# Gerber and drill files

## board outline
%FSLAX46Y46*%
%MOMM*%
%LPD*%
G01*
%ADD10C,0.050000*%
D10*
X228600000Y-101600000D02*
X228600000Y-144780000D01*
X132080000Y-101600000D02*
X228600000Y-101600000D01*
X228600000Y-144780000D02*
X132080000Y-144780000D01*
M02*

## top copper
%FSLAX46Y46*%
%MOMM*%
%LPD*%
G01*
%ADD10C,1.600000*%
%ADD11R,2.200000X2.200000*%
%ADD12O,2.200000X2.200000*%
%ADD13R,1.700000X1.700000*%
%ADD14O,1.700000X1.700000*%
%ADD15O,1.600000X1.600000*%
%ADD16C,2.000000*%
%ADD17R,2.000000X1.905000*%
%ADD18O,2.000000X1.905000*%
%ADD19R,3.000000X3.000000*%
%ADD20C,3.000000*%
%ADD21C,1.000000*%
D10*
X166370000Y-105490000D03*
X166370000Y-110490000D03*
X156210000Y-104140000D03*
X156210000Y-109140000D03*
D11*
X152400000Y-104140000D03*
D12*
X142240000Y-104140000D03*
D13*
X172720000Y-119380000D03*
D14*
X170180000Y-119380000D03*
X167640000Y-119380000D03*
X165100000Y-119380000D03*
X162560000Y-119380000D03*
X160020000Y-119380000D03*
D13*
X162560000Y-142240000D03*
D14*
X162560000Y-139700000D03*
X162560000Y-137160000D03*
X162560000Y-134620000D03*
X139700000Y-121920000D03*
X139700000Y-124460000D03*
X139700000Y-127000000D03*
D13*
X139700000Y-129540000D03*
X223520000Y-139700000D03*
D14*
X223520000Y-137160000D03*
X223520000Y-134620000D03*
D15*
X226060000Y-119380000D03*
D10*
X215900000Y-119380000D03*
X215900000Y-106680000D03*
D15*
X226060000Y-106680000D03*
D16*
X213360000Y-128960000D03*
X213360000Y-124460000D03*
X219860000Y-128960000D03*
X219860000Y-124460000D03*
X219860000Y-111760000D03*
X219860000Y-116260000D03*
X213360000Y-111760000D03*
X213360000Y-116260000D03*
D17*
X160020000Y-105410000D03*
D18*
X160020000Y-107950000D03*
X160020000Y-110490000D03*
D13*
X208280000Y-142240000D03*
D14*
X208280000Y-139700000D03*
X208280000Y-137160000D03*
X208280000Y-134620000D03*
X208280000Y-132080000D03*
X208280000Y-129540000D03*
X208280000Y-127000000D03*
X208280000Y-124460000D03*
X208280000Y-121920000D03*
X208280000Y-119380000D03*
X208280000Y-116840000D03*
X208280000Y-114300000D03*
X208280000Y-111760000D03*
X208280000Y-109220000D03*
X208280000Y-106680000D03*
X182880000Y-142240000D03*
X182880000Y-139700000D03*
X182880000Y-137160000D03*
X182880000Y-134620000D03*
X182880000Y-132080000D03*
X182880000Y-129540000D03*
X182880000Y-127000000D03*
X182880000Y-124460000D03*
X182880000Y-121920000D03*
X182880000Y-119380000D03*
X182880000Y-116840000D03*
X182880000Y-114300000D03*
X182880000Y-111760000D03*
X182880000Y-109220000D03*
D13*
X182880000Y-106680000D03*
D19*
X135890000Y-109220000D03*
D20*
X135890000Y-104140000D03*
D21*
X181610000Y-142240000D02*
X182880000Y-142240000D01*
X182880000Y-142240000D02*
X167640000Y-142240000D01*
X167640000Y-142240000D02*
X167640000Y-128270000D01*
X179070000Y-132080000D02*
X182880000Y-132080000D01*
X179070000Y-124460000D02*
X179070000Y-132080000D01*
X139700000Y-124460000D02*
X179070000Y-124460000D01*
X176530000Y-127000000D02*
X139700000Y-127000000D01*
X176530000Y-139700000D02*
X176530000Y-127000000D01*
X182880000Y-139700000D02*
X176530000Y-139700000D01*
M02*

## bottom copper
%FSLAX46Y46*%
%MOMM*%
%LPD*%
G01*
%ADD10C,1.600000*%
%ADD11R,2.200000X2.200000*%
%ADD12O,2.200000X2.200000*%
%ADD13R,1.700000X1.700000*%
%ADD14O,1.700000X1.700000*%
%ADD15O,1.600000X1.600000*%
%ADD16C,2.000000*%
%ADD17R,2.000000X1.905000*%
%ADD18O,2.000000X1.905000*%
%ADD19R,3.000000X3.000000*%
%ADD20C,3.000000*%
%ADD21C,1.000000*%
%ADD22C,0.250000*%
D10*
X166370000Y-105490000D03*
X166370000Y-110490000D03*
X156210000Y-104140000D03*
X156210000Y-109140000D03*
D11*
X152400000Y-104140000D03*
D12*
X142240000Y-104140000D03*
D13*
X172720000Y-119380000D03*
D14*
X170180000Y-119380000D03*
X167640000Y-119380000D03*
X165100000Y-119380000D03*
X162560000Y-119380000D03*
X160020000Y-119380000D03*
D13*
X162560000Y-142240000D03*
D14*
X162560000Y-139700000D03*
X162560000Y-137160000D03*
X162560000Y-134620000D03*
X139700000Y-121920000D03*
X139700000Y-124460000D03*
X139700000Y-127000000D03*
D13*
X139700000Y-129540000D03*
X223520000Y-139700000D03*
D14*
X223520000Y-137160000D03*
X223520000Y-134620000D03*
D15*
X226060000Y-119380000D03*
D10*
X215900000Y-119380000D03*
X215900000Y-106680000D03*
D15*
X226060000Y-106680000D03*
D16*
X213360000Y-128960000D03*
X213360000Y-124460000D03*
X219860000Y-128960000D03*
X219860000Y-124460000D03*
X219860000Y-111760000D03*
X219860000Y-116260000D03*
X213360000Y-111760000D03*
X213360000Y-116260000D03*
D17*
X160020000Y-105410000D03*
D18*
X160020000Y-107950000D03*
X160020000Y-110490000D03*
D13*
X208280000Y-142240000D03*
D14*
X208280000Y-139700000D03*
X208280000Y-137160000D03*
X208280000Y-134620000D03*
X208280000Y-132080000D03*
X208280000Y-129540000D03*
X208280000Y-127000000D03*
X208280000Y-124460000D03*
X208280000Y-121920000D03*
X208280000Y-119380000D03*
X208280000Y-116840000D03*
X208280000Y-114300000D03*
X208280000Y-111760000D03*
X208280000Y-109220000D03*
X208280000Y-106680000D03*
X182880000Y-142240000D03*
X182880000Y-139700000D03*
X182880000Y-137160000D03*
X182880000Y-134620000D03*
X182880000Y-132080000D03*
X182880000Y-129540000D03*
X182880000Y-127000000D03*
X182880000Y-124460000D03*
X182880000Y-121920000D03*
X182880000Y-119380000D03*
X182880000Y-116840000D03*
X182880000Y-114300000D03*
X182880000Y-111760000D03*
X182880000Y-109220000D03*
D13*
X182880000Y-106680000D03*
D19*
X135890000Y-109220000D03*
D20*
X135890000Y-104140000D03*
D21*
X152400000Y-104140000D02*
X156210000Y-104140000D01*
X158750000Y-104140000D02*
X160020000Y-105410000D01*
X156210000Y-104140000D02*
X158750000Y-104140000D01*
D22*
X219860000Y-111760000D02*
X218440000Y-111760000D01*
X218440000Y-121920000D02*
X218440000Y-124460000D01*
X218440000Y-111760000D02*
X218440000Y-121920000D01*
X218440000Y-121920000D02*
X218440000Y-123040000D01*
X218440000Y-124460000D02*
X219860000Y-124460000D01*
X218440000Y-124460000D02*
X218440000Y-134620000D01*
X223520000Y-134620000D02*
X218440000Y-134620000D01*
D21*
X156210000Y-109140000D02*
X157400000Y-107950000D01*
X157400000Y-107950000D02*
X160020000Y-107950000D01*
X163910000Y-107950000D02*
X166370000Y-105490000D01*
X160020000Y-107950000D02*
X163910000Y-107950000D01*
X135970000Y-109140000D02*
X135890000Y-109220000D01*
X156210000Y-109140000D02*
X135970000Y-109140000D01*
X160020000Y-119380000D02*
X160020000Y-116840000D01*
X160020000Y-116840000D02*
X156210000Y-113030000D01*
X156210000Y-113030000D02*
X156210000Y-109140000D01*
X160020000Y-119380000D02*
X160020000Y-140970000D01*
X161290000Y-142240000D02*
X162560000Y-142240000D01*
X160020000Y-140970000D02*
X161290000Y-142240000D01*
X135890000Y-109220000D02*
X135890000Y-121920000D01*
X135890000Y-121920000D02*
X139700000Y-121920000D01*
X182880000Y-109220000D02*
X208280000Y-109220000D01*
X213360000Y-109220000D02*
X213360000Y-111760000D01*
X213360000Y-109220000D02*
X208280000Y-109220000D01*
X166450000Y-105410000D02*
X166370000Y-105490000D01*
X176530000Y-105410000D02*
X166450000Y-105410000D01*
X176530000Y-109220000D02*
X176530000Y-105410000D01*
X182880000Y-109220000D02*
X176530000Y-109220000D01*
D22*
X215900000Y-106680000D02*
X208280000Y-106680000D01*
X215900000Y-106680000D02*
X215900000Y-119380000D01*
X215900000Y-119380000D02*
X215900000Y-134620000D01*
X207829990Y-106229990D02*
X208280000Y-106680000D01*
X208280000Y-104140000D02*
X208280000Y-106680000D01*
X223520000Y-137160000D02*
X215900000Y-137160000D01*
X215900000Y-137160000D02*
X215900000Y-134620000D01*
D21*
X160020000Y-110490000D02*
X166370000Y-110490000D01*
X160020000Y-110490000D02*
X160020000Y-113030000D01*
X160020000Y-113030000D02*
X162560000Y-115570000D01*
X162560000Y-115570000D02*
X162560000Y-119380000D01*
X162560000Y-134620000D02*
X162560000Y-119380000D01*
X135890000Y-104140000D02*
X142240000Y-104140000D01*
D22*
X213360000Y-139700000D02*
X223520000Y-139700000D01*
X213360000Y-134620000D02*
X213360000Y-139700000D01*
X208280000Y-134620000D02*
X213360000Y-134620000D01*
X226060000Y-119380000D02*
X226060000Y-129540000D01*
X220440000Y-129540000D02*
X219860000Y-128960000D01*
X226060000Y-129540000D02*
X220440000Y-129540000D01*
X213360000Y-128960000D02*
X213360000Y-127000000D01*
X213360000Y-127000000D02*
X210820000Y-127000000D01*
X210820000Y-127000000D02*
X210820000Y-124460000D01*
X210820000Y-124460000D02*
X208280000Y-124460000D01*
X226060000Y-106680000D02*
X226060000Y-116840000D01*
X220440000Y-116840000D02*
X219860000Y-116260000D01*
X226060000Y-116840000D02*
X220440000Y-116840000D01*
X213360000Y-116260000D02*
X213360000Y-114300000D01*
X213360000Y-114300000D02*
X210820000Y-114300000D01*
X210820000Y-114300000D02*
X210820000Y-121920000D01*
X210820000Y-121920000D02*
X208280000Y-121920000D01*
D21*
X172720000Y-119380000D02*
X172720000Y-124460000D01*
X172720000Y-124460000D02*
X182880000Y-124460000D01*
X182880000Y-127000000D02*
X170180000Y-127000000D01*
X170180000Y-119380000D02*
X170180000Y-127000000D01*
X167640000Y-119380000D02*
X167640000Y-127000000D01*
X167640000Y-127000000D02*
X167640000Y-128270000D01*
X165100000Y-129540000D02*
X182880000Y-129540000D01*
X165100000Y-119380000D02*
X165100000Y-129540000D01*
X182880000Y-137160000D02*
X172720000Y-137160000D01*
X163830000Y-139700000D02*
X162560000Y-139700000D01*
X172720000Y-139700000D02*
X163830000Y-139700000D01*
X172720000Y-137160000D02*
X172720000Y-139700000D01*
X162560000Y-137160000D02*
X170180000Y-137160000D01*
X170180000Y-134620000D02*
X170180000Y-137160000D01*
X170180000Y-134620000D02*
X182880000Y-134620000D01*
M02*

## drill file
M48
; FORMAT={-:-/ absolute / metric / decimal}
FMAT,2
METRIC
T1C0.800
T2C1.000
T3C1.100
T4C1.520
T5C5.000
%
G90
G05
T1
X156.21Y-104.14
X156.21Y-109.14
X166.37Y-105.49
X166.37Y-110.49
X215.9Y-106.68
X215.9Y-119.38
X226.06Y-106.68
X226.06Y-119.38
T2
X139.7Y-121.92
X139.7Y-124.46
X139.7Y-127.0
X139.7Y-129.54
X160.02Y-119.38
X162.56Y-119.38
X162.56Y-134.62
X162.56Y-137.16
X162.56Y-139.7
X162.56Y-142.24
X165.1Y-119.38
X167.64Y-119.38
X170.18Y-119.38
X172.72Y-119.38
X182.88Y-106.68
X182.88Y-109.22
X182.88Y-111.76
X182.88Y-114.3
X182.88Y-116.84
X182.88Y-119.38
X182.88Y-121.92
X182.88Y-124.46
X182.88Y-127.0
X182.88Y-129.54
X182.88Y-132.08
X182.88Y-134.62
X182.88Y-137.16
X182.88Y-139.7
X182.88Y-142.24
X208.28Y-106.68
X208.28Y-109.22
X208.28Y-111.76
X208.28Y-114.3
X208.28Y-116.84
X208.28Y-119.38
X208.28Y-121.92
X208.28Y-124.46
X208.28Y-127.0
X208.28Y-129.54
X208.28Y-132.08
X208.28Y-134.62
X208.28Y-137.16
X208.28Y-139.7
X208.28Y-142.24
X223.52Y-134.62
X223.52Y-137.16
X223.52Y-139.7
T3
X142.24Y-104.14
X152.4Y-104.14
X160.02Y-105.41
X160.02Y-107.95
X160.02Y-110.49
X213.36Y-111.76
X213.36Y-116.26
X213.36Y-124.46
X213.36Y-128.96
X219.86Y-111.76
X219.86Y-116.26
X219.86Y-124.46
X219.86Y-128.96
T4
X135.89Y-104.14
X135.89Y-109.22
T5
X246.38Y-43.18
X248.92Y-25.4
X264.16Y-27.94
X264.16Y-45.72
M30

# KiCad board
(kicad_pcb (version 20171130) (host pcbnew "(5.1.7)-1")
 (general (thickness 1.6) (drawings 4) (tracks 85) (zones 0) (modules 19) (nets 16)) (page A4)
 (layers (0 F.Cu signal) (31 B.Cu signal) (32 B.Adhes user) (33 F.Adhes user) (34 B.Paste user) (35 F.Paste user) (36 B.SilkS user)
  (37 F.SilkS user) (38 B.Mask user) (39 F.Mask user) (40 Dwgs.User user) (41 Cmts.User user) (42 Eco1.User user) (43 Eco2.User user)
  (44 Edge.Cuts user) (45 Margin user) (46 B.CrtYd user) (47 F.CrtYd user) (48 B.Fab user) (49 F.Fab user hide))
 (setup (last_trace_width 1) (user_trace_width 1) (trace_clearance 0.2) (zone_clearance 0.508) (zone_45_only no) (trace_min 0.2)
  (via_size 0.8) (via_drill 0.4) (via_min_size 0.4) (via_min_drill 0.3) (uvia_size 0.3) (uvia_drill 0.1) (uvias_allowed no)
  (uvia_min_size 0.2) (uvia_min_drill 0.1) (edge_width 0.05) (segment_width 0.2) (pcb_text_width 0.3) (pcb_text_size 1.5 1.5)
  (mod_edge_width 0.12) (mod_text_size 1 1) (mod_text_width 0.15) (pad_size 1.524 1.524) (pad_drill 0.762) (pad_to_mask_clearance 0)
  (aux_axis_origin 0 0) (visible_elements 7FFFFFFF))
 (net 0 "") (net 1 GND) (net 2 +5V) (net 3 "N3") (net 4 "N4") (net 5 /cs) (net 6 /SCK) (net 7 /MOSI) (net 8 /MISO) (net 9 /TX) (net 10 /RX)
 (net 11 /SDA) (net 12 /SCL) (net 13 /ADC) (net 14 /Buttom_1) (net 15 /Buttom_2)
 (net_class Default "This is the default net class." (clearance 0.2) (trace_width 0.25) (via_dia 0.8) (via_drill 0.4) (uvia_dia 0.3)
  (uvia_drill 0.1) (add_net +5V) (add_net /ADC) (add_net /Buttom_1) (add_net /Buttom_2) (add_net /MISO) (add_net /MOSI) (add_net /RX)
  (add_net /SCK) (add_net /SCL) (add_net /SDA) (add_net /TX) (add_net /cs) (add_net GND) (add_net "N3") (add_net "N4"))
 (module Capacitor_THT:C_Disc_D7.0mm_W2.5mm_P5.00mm (layer F.Cu) (at 166.37 110.49 90)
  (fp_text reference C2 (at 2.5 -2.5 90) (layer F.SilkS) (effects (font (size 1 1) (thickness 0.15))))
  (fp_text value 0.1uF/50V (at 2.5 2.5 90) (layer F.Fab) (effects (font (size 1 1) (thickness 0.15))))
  (pad 2 thru_hole circle (at 5 0 90) (size 1.6 1.6) (drill 0.8) (layers *.Cu *.Mask) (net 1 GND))
  (pad 1 thru_hole circle (at 0 0 90) (size 1.6 1.6) (drill 0.8) (layers *.Cu *.Mask) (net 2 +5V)))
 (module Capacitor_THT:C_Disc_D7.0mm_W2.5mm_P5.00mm (layer F.Cu) (at 156.21 104.14 270)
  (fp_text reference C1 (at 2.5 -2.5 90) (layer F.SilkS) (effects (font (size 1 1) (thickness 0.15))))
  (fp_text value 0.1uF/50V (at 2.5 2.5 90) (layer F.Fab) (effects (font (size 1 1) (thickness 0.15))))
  (pad 1 thru_hole circle (at 0 0 270) (size 1.6 1.6) (drill 0.8) (layers *.Cu *.Mask) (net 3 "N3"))
  (pad 2 thru_hole circle (at 5 0 270) (size 1.6 1.6) (drill 0.8) (layers *.Cu *.Mask) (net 1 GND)))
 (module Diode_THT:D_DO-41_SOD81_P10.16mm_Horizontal (layer F.Cu) (at 152.4 104.14 180)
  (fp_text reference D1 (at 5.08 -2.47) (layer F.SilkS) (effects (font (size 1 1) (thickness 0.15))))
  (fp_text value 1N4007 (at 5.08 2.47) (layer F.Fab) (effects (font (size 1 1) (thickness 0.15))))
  (pad 1 thru_hole rect (at 0 0 180) (size 2.2 2.2) (drill 1.1) (layers *.Cu *.Mask) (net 3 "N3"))
  (pad 2 thru_hole oval (at 10.16 0 180) (size 2.2 2.2) (drill 1.1) (layers *.Cu *.Mask) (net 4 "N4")))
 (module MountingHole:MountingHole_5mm (layer F.Cu) (at 248.92 25.4)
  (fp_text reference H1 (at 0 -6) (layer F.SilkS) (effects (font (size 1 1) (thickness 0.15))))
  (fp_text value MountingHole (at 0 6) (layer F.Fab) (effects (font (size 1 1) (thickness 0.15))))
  (pad 1 np_thru_hole circle (at 0 0) (size 5 5) (drill 5) (layers *.Cu *.Mask)))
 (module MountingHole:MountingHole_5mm (layer F.Cu) (at 264.16 45.72)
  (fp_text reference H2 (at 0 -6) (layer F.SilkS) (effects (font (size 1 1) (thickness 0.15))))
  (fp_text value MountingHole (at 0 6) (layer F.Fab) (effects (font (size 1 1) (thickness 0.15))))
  (pad 1 np_thru_hole circle (at 0 0) (size 5 5) (drill 5) (layers *.Cu *.Mask)))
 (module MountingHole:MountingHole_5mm (layer F.Cu) (at 264.16 27.94)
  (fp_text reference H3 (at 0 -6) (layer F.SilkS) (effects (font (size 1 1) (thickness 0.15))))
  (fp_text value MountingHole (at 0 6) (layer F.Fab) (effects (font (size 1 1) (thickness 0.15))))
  (pad 1 np_thru_hole circle (at 0 0) (size 5 5) (drill 5) (layers *.Cu *.Mask)))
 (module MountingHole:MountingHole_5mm (layer F.Cu) (at 246.38 43.18)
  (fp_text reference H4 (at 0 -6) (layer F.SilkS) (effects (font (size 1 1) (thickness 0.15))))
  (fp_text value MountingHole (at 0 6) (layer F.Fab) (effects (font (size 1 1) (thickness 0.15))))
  (pad 1 np_thru_hole circle (at 0 0) (size 5 5) (drill 5) (layers *.Cu *.Mask)))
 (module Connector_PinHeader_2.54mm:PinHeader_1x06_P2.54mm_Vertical (layer F.Cu) (at 172.72 119.38 270)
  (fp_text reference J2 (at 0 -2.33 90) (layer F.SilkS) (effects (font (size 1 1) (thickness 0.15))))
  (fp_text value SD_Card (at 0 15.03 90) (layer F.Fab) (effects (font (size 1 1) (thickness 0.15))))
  (pad 1 thru_hole rect (at 0 0 270) (size 1.7 1.7) (drill 1) (layers *.Cu *.Mask) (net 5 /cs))
  (pad 2 thru_hole oval (at 0 2.54 270) (size 1.7 1.7) (drill 1) (layers *.Cu *.Mask) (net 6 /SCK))
  (pad 3 thru_hole oval (at 0 5.08 270) (size 1.7 1.7) (drill 1) (layers *.Cu *.Mask) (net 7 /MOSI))
  (pad 4 thru_hole oval (at 0 7.62 270) (size 1.7 1.7) (drill 1) (layers *.Cu *.Mask) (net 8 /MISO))
  (pad 5 thru_hole oval (at 0 10.16 270) (size 1.7 1.7) (drill 1) (layers *.Cu *.Mask) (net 2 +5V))
  (pad 6 thru_hole oval (at 0 12.7 270) (size 1.7 1.7) (drill 1) (layers *.Cu *.Mask) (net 1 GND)))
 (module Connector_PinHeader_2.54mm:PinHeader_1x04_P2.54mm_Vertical (layer F.Cu) (at 162.56 142.24 180)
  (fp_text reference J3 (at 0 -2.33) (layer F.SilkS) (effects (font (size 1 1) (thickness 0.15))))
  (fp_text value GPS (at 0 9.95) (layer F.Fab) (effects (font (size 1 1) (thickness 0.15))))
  (pad 1 thru_hole rect (at 0 0 180) (size 1.7 1.7) (drill 1) (layers *.Cu *.Mask) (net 1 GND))
  (pad 2 thru_hole oval (at 0 2.54 180) (size 1.7 1.7) (drill 1) (layers *.Cu *.Mask) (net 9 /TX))
  (pad 3 thru_hole oval (at 0 5.08 180) (size 1.7 1.7) (drill 1) (layers *.Cu *.Mask) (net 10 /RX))
  (pad 4 thru_hole oval (at 0 7.62 180) (size 1.7 1.7) (drill 1) (layers *.Cu *.Mask) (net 2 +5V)))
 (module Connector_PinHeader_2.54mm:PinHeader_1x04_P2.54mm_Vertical (layer F.Cu) (at 139.7 129.54 180)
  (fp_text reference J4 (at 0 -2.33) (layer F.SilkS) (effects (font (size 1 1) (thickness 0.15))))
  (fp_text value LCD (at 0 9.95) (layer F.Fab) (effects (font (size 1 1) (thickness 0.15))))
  (pad 4 thru_hole oval (at 0 7.62 180) (size 1.7 1.7) (drill 1) (layers *.Cu *.Mask) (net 1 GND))
  (pad 3 thru_hole oval (at 0 5.08 180) (size 1.7 1.7) (drill 1) (layers *.Cu *.Mask) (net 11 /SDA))
  (pad 2 thru_hole oval (at 0 2.54 180) (size 1.7 1.7) (drill 1) (layers *.Cu *.Mask) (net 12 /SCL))
  (pad 1 thru_hole rect (at 0 0 180) (size 1.7 1.7) (drill 1) (layers *.Cu *.Mask) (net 2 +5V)))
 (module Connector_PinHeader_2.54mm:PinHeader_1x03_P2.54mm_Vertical (layer F.Cu) (at 223.52 139.7 180)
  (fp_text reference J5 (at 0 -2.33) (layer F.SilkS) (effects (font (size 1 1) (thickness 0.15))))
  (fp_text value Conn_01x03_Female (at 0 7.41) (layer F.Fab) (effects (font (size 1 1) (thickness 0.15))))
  (pad 1 thru_hole rect (at 0 0 180) (size 1.7 1.7) (drill 1) (layers *.Cu *.Mask) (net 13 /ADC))
  (pad 2 thru_hole oval (at 0 2.54 180) (size 1.7 1.7) (drill 1) (layers *.Cu *.Mask) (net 2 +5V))
  (pad 3 thru_hole oval (at 0 5.08 180) (size 1.7 1.7) (drill 1) (layers *.Cu *.Mask) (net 1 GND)))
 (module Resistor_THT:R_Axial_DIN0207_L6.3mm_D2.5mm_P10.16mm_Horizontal (layer F.Cu) (at 215.9 119.38)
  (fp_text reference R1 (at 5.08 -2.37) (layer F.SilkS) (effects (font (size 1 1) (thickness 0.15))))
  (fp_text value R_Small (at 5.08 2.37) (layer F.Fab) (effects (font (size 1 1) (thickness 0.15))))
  (pad 2 thru_hole oval (at 10.16 0) (size 1.6 1.6) (drill 0.8) (layers *.Cu *.Mask) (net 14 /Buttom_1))
  (pad 1 thru_hole circle (at 0 0) (size 1.6 1.6) (drill 0.8) (layers *.Cu *.Mask) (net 2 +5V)))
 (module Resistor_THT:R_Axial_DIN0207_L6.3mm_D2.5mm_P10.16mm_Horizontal (layer F.Cu) (at 215.9 106.68)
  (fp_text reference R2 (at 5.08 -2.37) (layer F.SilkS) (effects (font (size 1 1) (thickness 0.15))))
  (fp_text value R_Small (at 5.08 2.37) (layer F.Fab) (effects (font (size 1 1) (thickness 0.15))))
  (pad 1 thru_hole circle (at 0 0) (size 1.6 1.6) (drill 0.8) (layers *.Cu *.Mask) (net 2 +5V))
  (pad 2 thru_hole oval (at 10.16 0) (size 1.6 1.6) (drill 0.8) (layers *.Cu *.Mask) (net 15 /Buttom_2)))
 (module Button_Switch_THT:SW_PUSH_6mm (layer F.Cu) (at 213.36 124.46)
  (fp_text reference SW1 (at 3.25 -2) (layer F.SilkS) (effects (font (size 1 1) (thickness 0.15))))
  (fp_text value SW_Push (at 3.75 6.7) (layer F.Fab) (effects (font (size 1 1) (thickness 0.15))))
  (pad 2 thru_hole circle (at 0 4.5 90) (size 2 2) (drill 1.1) (layers *.Cu *.Mask) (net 14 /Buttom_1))
  (pad 1 thru_hole circle (at 0 0 90) (size 2 2) (drill 1.1) (layers *.Cu *.Mask) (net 1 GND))
  (pad 2 thru_hole circle (at 6.5 4.5 90) (size 2 2) (drill 1.1) (layers *.Cu *.Mask) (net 14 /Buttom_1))
  (pad 1 thru_hole circle (at 6.5 0 90) (size 2 2) (drill 1.1) (layers *.Cu *.Mask) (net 1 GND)))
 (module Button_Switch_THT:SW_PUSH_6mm (layer F.Cu) (at 213.36 111.76)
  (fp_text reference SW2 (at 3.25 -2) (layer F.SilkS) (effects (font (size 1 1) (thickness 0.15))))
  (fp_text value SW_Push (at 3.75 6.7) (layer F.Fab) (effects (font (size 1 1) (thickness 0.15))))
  (pad 1 thru_hole circle (at 6.5 0 90) (size 2 2) (drill 1.1) (layers *.Cu *.Mask) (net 1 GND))
  (pad 2 thru_hole circle (at 6.5 4.5 90) (size 2 2) (drill 1.1) (layers *.Cu *.Mask) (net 15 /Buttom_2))
  (pad 1 thru_hole circle (at 0 0 90) (size 2 2) (drill 1.1) (layers *.Cu *.Mask) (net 1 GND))
  (pad 2 thru_hole circle (at 0 4.5 90) (size 2 2) (drill 1.1) (layers *.Cu *.Mask) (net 15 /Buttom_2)))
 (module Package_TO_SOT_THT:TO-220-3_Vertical (layer F.Cu) (at 160.02 105.41 270)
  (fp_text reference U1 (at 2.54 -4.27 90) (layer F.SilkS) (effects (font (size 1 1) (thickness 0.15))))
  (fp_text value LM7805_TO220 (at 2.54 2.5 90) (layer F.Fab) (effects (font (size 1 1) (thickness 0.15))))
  (pad 1 thru_hole rect (at 0 0 270) (size 1.905 2) (drill 1.1) (layers *.Cu *.Mask) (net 3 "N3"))
  (pad 2 thru_hole oval (at 2.54 0 270) (size 1.905 2) (drill 1.1) (layers *.Cu *.Mask) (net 1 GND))
  (pad 3 thru_hole oval (at 5.08 0 270) (size 1.905 2) (drill 1.1) (layers *.Cu *.Mask) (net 2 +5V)))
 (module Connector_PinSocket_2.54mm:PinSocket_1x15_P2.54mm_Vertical (layer F.Cu) (at 208.28 142.24 180)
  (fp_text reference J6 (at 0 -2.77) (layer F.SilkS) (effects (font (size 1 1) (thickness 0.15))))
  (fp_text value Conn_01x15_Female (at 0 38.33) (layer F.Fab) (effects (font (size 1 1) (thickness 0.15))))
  (pad 1 thru_hole rect (at 0 0 180) (size 1.7 1.7) (drill 1) (layers *.Cu *.Mask))
  (pad 2 thru_hole oval (at 0 2.54 180) (size 1.7 1.7) (drill 1) (layers *.Cu *.Mask))
  (pad 3 thru_hole oval (at 0 5.08 180) (size 1.7 1.7) (drill 1) (layers *.Cu *.Mask))
  (pad 4 thru_hole oval (at 0 7.62 180) (size 1.7 1.7) (drill 1) (layers *.Cu *.Mask) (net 13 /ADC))
  (pad 5 thru_hole oval (at 0 10.16 180) (size 1.7 1.7) (drill 1) (layers *.Cu *.Mask))
  (pad 6 thru_hole oval (at 0 12.7 180) (size 1.7 1.7) (drill 1) (layers *.Cu *.Mask))
  (pad 7 thru_hole oval (at 0 15.24 180) (size 1.7 1.7) (drill 1) (layers *.Cu *.Mask))
  (pad 8 thru_hole oval (at 0 17.78 180) (size 1.7 1.7) (drill 1) (layers *.Cu *.Mask) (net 14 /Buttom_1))
  (pad 9 thru_hole oval (at 0 20.32 180) (size 1.7 1.7) (drill 1) (layers *.Cu *.Mask) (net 15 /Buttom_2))
  (pad 10 thru_hole oval (at 0 22.86 180) (size 1.7 1.7) (drill 1) (layers *.Cu *.Mask))
  (pad 11 thru_hole oval (at 0 25.4 180) (size 1.7 1.7) (drill 1) (layers *.Cu *.Mask))
  (pad 12 thru_hole oval (at 0 27.94 180) (size 1.7 1.7) (drill 1) (layers *.Cu *.Mask))
  (pad 13 thru_hole oval (at 0 30.48 180) (size 1.7 1.7) (drill 1) (layers *.Cu *.Mask))
  (pad 14 thru_hole oval (at 0 33.02 180) (size 1.7 1.7) (drill 1) (layers *.Cu *.Mask) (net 1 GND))
  (pad 15 thru_hole oval (at 0 35.56 180) (size 1.7 1.7) (drill 1) (layers *.Cu *.Mask) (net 2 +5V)))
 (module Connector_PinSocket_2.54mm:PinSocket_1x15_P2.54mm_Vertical (layer F.Cu) (at 182.88 106.68)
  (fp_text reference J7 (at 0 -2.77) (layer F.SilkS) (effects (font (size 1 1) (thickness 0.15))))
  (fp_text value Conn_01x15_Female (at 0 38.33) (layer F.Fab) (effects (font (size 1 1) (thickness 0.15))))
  (pad 15 thru_hole oval (at 0 35.56) (size 1.7 1.7) (drill 1) (layers *.Cu *.Mask) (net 7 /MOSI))
  (pad 14 thru_hole oval (at 0 33.02) (size 1.7 1.7) (drill 1) (layers *.Cu *.Mask) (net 12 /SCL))
  (pad 13 thru_hole oval (at 0 30.48) (size 1.7 1.7) (drill 1) (layers *.Cu *.Mask) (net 9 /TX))
  (pad 12 thru_hole oval (at 0 27.94) (size 1.7 1.7) (drill 1) (layers *.Cu *.Mask) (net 10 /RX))
  (pad 11 thru_hole oval (at 0 25.4) (size 1.7 1.7) (drill 1) (layers *.Cu *.Mask) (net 11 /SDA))
  (pad 10 thru_hole oval (at 0 22.86) (size 1.7 1.7) (drill 1) (layers *.Cu *.Mask) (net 8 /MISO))
  (pad 9 thru_hole oval (at 0 20.32) (size 1.7 1.7) (drill 1) (layers *.Cu *.Mask) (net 6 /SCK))
  (pad 8 thru_hole oval (at 0 17.78) (size 1.7 1.7) (drill 1) (layers *.Cu *.Mask) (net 5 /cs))
  (pad 7 thru_hole oval (at 0 15.24) (size 1.7 1.7) (drill 1) (layers *.Cu *.Mask))
  (pad 6 thru_hole oval (at 0 12.7) (size 1.7 1.7) (drill 1) (layers *.Cu *.Mask))
  (pad 5 thru_hole oval (at 0 10.16) (size 1.7 1.7) (drill 1) (layers *.Cu *.Mask))
  (pad 4 thru_hole oval (at 0 7.62) (size 1.7 1.7) (drill 1) (layers *.Cu *.Mask))
  (pad 3 thru_hole oval (at 0 5.08) (size 1.7 1.7) (drill 1) (layers *.Cu *.Mask))
  (pad 2 thru_hole oval (at 0 2.54) (size 1.7 1.7) (drill 1) (layers *.Cu *.Mask) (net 1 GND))
  (pad 1 thru_hole rect (at 0 0) (size 1.7 1.7) (drill 1) (layers *.Cu *.Mask)))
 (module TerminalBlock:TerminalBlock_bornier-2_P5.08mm (layer F.Cu) (at 135.89 109.22 90)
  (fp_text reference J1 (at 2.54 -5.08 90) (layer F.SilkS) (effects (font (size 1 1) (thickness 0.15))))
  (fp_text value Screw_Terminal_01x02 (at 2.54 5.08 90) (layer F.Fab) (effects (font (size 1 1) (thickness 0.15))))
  (pad 1 thru_hole rect (at 0 0 90) (size 3 3) (drill 1.52) (layers *.Cu *.Mask) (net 1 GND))
  (pad 2 thru_hole circle (at 5.08 0 90) (size 3 3) (drill 1.52) (layers *.Cu *.Mask) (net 4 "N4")))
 (gr_line (start 228.6 101.6) (end 228.6 144.78) (layer Edge.Cuts) (width 0.05))
 (gr_line (start 132.08 101.6) (end 228.6 101.6) (layer Edge.Cuts) (width 0.05))
 (gr_line (start 228.6 144.78) (end 132.08 144.78) (layer Edge.Cuts) (width 0.05))
 (segment (start 152.4 104.14) (end 156.21 104.14) (width 1) (layer B.Cu) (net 3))
 (segment (start 158.75 104.14) (end 160.02 105.41) (width 1) (layer B.Cu) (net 3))
 (segment (start 156.21 104.14) (end 158.75 104.14) (width 1) (layer B.Cu) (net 3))
 (segment (start 219.86 111.76) (end 218.44 111.76) (width 0.25) (layer B.Cu) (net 1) (status 10))
 (segment (start 218.44 121.92) (end 218.44 124.46) (width 0.25) (layer B.Cu) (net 1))
 (segment (start 218.44 111.76) (end 218.44 121.92) (width 0.25) (layer B.Cu) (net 1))
 (segment (start 218.44 121.92) (end 218.44 123.04) (width 0.25) (layer B.Cu) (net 1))
 (segment (start 218.44 124.46) (end 219.86 124.46) (width 0.25) (layer B.Cu) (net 1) (status 20))
 (segment (start 218.44 124.46) (end 218.44 134.62) (width 0.25) (layer B.Cu) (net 1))
 (segment (start 223.52 134.62) (end 218.44 134.62) (width 0.25) (layer B.Cu) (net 1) (status 10))
 (segment (start 156.21 109.14) (end 157.4 107.95) (width 1) (layer B.Cu) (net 1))
 (segment (start 157.4 107.95) (end 160.02 107.95) (width 1) (layer B.Cu) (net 1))
 (segment (start 163.91 107.95) (end 166.37 105.49) (width 1) (layer B.Cu) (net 1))
 (segment (start 160.02 107.95) (end 163.91 107.95) (width 1) (layer B.Cu) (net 1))
 (segment (start 135.97 109.14) (end 135.89 109.22) (width 1) (layer B.Cu) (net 1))
 (segment (start 156.21 109.14) (end 135.97 109.14) (width 1) (layer B.Cu) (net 1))
 (segment (start 160.02 119.38) (end 160.02 116.84) (width 1) (layer B.Cu) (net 1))
 (segment (start 160.02 116.84) (end 156.21 113.03) (width 1) (layer B.Cu) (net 1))
 (segment (start 156.21 113.03) (end 156.21 109.14) (width 1) (layer B.Cu) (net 1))
 (segment (start 160.02 119.38) (end 160.02 140.97) (width 1) (layer B.Cu) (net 1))
 (segment (start 161.29 142.24) (end 162.56 142.24) (width 1) (layer B.Cu) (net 1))
 (segment (start 160.02 140.97) (end 161.29 142.24) (width 1) (layer B.Cu) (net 1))
 (segment (start 135.89 109.22) (end 135.89 121.92) (width 1) (layer B.Cu) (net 1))
 (segment (start 135.89 121.92) (end 139.7 121.92) (width 1) (layer B.Cu) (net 1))
 (segment (start 182.88 109.22) (end 208.28 109.22) (width 1) (layer B.Cu) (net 1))
 (segment (start 213.36 109.22) (end 213.36 111.76) (width 1) (layer B.Cu) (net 1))
 (segment (start 213.36 109.22) (end 208.28 109.22) (width 1) (layer B.Cu) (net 1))
 (segment (start 166.45 105.41) (end 166.37 105.49) (width 1) (layer B.Cu) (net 1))
 (segment (start 176.53 105.41) (end 166.45 105.41) (width 1) (layer B.Cu) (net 1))
 (segment (start 176.53 109.22) (end 176.53 105.41) (width 1) (layer B.Cu) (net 1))
 (segment (start 182.88 109.22) (end 176.53 109.22) (width 1) (layer B.Cu) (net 1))
 (segment (start 215.9 106.68) (end 208.28 106.68) (width 0.25) (layer B.Cu) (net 2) (status 30))
 (segment (start 215.9 106.68) (end 215.9 119.38) (width 0.25) (layer B.Cu) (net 2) (status 30))
 (segment (start 215.9 119.38) (end 215.9 134.62) (width 0.25) (layer B.Cu) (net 2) (status 10))
 (segment (start 207.82999 106.22999) (end 208.28 106.68) (width 0.25) (layer B.Cu) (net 2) (status 30))
 (segment (start 208.28 104.14) (end 208.28 106.68) (width 0.25) (layer B.Cu) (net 2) (status 20))
 (segment (start 223.52 137.16) (end 215.9 137.16) (width 0.25) (layer B.Cu) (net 2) (status 10))
 (segment (start 215.9 137.16) (end 215.9 134.62) (width 0.25) (layer B.Cu) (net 2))
 (segment (start 160.02 110.49) (end 166.37 110.49) (width 1) (layer B.Cu) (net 2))
 (segment (start 160.02 110.49) (end 160.02 113.03) (width 1) (layer B.Cu) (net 2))
 (segment (start 160.02 113.03) (end 162.56 115.57) (width 1) (layer B.Cu) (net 2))
 (segment (start 162.56 115.57) (end 162.56 119.38) (width 1) (layer B.Cu) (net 2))
 (segment (start 162.56 134.62) (end 162.56 119.38) (width 1) (layer B.Cu) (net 2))
 (segment (start 135.89 104.14) (end 142.24 104.14) (width 1) (layer B.Cu) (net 4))
 (segment (start 213.36 139.7) (end 223.52 139.7) (width 0.25) (layer B.Cu) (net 13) (status 20))
 (segment (start 213.36 134.62) (end 213.36 139.7) (width 0.25) (layer B.Cu) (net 13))
 (segment (start 208.28 134.62) (end 213.36 134.62) (width 0.25) (layer B.Cu) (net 13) (status 10))
 (segment (start 226.06 119.38) (end 226.06 129.54) (width 0.25) (layer B.Cu) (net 14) (status 10))
 (segment (start 220.44 129.54) (end 219.86 128.96) (width 0.25) (layer B.Cu) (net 14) (status 30))
 (segment (start 226.06 129.54) (end 220.44 129.54) (width 0.25) (layer B.Cu) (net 14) (status 20))
 (segment (start 213.36 128.96) (end 213.36 127) (width 0.25) (layer B.Cu) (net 14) (status 10))
 (segment (start 213.36 127) (end 210.82 127) (width 0.25) (layer B.Cu) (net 14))
 (segment (start 210.82 127) (end 210.82 124.46) (width 0.25) (layer B.Cu) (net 14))
 (segment (start 210.82 124.46) (end 208.28 124.46) (width 0.25) (layer B.Cu) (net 14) (status 20))
 (segment (start 226.06 106.68) (end 226.06 116.84) (width 0.25) (layer B.Cu) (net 15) (status 10))
 (segment (start 220.44 116.84) (end 219.86 116.26) (width 0.25) (layer B.Cu) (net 15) (status 30))
 (segment (start 226.06 116.84) (end 220.44 116.84) (width 0.25) (layer B.Cu) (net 15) (status 20))
 (segment (start 213.36 116.26) (end 213.36 114.3) (width 0.25) (layer B.Cu) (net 15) (status 10))
 (segment (start 213.36 114.3) (end 210.82 114.3) (width 0.25) (layer B.Cu) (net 15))
 (segment (start 210.82 114.3) (end 210.82 121.92) (width 0.25) (layer B.Cu) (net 15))
 (segment (start 210.82 121.92) (end 208.28 121.92) (width 0.25) (layer B.Cu) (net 15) (status 20))
 (segment (start 172.72 119.38) (end 172.72 124.46) (width 1) (layer B.Cu) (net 5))
 (segment (start 172.72 124.46) (end 182.88 124.46) (width 1) (layer B.Cu) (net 5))
 (segment (start 182.88 127) (end 170.18 127) (width 1) (layer B.Cu) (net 6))
 (segment (start 170.18 119.38) (end 170.18 127) (width 1) (layer B.Cu) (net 6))
 (segment (start 181.61 142.24) (end 182.88 142.24) (width 1) (layer F.Cu) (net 7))
 (segment (start 167.64 119.38) (end 167.64 127) (width 1) (layer B.Cu) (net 7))
 (segment (start 182.88 142.24) (end 167.64 142.24) (width 1) (layer F.Cu) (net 7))
 (segment (start 167.64 142.24) (end 167.64 128.27) (width 1) (layer F.Cu) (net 7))
 (segment (start 167.64 127) (end 167.64 128.27) (width 1) (layer B.Cu) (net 7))
 (segment (start 165.1 129.54) (end 182.88 129.54) (width 1) (layer B.Cu) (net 8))
 (segment (start 165.1 119.38) (end 165.1 129.54) (width 1) (layer B.Cu) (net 8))
 (segment (start 182.88 137.16) (end 172.72 137.16) (width 1) (layer B.Cu) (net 9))
 (segment (start 163.83 139.7) (end 162.56 139.7) (width 1) (layer B.Cu) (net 9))
 (segment (start 172.72 139.7) (end 163.83 139.7) (width 1) (layer B.Cu) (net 9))
 (segment (start 172.72 137.16) (end 172.72 139.7) (width 1) (layer B.Cu) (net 9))
 (segment (start 162.56 137.16) (end 170.18 137.16) (width 1) (layer B.Cu) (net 10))
 (segment (start 170.18 134.62) (end 170.18 137.16) (width 1) (layer B.Cu) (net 10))
 (segment (start 170.18 134.62) (end 182.88 134.62) (width 1) (layer B.Cu) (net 10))
 (segment (start 179.07 132.08) (end 182.88 132.08) (width 1) (layer F.Cu) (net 11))
 (segment (start 179.07 124.46) (end 179.07 132.08) (width 1) (layer F.Cu) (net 11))
 (segment (start 139.7 124.46) (end 179.07 124.46) (width 1) (layer F.Cu) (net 11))
 (segment (start 176.53 127) (end 139.7 127) (width 1) (layer F.Cu) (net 12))
 (segment (start 176.53 139.7) (end 176.53 127) (width 1) (layer F.Cu) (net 12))
 (segment (start 182.88 139.7) (end 176.53 139.7) (width 1) (layer F.Cu) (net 12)))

